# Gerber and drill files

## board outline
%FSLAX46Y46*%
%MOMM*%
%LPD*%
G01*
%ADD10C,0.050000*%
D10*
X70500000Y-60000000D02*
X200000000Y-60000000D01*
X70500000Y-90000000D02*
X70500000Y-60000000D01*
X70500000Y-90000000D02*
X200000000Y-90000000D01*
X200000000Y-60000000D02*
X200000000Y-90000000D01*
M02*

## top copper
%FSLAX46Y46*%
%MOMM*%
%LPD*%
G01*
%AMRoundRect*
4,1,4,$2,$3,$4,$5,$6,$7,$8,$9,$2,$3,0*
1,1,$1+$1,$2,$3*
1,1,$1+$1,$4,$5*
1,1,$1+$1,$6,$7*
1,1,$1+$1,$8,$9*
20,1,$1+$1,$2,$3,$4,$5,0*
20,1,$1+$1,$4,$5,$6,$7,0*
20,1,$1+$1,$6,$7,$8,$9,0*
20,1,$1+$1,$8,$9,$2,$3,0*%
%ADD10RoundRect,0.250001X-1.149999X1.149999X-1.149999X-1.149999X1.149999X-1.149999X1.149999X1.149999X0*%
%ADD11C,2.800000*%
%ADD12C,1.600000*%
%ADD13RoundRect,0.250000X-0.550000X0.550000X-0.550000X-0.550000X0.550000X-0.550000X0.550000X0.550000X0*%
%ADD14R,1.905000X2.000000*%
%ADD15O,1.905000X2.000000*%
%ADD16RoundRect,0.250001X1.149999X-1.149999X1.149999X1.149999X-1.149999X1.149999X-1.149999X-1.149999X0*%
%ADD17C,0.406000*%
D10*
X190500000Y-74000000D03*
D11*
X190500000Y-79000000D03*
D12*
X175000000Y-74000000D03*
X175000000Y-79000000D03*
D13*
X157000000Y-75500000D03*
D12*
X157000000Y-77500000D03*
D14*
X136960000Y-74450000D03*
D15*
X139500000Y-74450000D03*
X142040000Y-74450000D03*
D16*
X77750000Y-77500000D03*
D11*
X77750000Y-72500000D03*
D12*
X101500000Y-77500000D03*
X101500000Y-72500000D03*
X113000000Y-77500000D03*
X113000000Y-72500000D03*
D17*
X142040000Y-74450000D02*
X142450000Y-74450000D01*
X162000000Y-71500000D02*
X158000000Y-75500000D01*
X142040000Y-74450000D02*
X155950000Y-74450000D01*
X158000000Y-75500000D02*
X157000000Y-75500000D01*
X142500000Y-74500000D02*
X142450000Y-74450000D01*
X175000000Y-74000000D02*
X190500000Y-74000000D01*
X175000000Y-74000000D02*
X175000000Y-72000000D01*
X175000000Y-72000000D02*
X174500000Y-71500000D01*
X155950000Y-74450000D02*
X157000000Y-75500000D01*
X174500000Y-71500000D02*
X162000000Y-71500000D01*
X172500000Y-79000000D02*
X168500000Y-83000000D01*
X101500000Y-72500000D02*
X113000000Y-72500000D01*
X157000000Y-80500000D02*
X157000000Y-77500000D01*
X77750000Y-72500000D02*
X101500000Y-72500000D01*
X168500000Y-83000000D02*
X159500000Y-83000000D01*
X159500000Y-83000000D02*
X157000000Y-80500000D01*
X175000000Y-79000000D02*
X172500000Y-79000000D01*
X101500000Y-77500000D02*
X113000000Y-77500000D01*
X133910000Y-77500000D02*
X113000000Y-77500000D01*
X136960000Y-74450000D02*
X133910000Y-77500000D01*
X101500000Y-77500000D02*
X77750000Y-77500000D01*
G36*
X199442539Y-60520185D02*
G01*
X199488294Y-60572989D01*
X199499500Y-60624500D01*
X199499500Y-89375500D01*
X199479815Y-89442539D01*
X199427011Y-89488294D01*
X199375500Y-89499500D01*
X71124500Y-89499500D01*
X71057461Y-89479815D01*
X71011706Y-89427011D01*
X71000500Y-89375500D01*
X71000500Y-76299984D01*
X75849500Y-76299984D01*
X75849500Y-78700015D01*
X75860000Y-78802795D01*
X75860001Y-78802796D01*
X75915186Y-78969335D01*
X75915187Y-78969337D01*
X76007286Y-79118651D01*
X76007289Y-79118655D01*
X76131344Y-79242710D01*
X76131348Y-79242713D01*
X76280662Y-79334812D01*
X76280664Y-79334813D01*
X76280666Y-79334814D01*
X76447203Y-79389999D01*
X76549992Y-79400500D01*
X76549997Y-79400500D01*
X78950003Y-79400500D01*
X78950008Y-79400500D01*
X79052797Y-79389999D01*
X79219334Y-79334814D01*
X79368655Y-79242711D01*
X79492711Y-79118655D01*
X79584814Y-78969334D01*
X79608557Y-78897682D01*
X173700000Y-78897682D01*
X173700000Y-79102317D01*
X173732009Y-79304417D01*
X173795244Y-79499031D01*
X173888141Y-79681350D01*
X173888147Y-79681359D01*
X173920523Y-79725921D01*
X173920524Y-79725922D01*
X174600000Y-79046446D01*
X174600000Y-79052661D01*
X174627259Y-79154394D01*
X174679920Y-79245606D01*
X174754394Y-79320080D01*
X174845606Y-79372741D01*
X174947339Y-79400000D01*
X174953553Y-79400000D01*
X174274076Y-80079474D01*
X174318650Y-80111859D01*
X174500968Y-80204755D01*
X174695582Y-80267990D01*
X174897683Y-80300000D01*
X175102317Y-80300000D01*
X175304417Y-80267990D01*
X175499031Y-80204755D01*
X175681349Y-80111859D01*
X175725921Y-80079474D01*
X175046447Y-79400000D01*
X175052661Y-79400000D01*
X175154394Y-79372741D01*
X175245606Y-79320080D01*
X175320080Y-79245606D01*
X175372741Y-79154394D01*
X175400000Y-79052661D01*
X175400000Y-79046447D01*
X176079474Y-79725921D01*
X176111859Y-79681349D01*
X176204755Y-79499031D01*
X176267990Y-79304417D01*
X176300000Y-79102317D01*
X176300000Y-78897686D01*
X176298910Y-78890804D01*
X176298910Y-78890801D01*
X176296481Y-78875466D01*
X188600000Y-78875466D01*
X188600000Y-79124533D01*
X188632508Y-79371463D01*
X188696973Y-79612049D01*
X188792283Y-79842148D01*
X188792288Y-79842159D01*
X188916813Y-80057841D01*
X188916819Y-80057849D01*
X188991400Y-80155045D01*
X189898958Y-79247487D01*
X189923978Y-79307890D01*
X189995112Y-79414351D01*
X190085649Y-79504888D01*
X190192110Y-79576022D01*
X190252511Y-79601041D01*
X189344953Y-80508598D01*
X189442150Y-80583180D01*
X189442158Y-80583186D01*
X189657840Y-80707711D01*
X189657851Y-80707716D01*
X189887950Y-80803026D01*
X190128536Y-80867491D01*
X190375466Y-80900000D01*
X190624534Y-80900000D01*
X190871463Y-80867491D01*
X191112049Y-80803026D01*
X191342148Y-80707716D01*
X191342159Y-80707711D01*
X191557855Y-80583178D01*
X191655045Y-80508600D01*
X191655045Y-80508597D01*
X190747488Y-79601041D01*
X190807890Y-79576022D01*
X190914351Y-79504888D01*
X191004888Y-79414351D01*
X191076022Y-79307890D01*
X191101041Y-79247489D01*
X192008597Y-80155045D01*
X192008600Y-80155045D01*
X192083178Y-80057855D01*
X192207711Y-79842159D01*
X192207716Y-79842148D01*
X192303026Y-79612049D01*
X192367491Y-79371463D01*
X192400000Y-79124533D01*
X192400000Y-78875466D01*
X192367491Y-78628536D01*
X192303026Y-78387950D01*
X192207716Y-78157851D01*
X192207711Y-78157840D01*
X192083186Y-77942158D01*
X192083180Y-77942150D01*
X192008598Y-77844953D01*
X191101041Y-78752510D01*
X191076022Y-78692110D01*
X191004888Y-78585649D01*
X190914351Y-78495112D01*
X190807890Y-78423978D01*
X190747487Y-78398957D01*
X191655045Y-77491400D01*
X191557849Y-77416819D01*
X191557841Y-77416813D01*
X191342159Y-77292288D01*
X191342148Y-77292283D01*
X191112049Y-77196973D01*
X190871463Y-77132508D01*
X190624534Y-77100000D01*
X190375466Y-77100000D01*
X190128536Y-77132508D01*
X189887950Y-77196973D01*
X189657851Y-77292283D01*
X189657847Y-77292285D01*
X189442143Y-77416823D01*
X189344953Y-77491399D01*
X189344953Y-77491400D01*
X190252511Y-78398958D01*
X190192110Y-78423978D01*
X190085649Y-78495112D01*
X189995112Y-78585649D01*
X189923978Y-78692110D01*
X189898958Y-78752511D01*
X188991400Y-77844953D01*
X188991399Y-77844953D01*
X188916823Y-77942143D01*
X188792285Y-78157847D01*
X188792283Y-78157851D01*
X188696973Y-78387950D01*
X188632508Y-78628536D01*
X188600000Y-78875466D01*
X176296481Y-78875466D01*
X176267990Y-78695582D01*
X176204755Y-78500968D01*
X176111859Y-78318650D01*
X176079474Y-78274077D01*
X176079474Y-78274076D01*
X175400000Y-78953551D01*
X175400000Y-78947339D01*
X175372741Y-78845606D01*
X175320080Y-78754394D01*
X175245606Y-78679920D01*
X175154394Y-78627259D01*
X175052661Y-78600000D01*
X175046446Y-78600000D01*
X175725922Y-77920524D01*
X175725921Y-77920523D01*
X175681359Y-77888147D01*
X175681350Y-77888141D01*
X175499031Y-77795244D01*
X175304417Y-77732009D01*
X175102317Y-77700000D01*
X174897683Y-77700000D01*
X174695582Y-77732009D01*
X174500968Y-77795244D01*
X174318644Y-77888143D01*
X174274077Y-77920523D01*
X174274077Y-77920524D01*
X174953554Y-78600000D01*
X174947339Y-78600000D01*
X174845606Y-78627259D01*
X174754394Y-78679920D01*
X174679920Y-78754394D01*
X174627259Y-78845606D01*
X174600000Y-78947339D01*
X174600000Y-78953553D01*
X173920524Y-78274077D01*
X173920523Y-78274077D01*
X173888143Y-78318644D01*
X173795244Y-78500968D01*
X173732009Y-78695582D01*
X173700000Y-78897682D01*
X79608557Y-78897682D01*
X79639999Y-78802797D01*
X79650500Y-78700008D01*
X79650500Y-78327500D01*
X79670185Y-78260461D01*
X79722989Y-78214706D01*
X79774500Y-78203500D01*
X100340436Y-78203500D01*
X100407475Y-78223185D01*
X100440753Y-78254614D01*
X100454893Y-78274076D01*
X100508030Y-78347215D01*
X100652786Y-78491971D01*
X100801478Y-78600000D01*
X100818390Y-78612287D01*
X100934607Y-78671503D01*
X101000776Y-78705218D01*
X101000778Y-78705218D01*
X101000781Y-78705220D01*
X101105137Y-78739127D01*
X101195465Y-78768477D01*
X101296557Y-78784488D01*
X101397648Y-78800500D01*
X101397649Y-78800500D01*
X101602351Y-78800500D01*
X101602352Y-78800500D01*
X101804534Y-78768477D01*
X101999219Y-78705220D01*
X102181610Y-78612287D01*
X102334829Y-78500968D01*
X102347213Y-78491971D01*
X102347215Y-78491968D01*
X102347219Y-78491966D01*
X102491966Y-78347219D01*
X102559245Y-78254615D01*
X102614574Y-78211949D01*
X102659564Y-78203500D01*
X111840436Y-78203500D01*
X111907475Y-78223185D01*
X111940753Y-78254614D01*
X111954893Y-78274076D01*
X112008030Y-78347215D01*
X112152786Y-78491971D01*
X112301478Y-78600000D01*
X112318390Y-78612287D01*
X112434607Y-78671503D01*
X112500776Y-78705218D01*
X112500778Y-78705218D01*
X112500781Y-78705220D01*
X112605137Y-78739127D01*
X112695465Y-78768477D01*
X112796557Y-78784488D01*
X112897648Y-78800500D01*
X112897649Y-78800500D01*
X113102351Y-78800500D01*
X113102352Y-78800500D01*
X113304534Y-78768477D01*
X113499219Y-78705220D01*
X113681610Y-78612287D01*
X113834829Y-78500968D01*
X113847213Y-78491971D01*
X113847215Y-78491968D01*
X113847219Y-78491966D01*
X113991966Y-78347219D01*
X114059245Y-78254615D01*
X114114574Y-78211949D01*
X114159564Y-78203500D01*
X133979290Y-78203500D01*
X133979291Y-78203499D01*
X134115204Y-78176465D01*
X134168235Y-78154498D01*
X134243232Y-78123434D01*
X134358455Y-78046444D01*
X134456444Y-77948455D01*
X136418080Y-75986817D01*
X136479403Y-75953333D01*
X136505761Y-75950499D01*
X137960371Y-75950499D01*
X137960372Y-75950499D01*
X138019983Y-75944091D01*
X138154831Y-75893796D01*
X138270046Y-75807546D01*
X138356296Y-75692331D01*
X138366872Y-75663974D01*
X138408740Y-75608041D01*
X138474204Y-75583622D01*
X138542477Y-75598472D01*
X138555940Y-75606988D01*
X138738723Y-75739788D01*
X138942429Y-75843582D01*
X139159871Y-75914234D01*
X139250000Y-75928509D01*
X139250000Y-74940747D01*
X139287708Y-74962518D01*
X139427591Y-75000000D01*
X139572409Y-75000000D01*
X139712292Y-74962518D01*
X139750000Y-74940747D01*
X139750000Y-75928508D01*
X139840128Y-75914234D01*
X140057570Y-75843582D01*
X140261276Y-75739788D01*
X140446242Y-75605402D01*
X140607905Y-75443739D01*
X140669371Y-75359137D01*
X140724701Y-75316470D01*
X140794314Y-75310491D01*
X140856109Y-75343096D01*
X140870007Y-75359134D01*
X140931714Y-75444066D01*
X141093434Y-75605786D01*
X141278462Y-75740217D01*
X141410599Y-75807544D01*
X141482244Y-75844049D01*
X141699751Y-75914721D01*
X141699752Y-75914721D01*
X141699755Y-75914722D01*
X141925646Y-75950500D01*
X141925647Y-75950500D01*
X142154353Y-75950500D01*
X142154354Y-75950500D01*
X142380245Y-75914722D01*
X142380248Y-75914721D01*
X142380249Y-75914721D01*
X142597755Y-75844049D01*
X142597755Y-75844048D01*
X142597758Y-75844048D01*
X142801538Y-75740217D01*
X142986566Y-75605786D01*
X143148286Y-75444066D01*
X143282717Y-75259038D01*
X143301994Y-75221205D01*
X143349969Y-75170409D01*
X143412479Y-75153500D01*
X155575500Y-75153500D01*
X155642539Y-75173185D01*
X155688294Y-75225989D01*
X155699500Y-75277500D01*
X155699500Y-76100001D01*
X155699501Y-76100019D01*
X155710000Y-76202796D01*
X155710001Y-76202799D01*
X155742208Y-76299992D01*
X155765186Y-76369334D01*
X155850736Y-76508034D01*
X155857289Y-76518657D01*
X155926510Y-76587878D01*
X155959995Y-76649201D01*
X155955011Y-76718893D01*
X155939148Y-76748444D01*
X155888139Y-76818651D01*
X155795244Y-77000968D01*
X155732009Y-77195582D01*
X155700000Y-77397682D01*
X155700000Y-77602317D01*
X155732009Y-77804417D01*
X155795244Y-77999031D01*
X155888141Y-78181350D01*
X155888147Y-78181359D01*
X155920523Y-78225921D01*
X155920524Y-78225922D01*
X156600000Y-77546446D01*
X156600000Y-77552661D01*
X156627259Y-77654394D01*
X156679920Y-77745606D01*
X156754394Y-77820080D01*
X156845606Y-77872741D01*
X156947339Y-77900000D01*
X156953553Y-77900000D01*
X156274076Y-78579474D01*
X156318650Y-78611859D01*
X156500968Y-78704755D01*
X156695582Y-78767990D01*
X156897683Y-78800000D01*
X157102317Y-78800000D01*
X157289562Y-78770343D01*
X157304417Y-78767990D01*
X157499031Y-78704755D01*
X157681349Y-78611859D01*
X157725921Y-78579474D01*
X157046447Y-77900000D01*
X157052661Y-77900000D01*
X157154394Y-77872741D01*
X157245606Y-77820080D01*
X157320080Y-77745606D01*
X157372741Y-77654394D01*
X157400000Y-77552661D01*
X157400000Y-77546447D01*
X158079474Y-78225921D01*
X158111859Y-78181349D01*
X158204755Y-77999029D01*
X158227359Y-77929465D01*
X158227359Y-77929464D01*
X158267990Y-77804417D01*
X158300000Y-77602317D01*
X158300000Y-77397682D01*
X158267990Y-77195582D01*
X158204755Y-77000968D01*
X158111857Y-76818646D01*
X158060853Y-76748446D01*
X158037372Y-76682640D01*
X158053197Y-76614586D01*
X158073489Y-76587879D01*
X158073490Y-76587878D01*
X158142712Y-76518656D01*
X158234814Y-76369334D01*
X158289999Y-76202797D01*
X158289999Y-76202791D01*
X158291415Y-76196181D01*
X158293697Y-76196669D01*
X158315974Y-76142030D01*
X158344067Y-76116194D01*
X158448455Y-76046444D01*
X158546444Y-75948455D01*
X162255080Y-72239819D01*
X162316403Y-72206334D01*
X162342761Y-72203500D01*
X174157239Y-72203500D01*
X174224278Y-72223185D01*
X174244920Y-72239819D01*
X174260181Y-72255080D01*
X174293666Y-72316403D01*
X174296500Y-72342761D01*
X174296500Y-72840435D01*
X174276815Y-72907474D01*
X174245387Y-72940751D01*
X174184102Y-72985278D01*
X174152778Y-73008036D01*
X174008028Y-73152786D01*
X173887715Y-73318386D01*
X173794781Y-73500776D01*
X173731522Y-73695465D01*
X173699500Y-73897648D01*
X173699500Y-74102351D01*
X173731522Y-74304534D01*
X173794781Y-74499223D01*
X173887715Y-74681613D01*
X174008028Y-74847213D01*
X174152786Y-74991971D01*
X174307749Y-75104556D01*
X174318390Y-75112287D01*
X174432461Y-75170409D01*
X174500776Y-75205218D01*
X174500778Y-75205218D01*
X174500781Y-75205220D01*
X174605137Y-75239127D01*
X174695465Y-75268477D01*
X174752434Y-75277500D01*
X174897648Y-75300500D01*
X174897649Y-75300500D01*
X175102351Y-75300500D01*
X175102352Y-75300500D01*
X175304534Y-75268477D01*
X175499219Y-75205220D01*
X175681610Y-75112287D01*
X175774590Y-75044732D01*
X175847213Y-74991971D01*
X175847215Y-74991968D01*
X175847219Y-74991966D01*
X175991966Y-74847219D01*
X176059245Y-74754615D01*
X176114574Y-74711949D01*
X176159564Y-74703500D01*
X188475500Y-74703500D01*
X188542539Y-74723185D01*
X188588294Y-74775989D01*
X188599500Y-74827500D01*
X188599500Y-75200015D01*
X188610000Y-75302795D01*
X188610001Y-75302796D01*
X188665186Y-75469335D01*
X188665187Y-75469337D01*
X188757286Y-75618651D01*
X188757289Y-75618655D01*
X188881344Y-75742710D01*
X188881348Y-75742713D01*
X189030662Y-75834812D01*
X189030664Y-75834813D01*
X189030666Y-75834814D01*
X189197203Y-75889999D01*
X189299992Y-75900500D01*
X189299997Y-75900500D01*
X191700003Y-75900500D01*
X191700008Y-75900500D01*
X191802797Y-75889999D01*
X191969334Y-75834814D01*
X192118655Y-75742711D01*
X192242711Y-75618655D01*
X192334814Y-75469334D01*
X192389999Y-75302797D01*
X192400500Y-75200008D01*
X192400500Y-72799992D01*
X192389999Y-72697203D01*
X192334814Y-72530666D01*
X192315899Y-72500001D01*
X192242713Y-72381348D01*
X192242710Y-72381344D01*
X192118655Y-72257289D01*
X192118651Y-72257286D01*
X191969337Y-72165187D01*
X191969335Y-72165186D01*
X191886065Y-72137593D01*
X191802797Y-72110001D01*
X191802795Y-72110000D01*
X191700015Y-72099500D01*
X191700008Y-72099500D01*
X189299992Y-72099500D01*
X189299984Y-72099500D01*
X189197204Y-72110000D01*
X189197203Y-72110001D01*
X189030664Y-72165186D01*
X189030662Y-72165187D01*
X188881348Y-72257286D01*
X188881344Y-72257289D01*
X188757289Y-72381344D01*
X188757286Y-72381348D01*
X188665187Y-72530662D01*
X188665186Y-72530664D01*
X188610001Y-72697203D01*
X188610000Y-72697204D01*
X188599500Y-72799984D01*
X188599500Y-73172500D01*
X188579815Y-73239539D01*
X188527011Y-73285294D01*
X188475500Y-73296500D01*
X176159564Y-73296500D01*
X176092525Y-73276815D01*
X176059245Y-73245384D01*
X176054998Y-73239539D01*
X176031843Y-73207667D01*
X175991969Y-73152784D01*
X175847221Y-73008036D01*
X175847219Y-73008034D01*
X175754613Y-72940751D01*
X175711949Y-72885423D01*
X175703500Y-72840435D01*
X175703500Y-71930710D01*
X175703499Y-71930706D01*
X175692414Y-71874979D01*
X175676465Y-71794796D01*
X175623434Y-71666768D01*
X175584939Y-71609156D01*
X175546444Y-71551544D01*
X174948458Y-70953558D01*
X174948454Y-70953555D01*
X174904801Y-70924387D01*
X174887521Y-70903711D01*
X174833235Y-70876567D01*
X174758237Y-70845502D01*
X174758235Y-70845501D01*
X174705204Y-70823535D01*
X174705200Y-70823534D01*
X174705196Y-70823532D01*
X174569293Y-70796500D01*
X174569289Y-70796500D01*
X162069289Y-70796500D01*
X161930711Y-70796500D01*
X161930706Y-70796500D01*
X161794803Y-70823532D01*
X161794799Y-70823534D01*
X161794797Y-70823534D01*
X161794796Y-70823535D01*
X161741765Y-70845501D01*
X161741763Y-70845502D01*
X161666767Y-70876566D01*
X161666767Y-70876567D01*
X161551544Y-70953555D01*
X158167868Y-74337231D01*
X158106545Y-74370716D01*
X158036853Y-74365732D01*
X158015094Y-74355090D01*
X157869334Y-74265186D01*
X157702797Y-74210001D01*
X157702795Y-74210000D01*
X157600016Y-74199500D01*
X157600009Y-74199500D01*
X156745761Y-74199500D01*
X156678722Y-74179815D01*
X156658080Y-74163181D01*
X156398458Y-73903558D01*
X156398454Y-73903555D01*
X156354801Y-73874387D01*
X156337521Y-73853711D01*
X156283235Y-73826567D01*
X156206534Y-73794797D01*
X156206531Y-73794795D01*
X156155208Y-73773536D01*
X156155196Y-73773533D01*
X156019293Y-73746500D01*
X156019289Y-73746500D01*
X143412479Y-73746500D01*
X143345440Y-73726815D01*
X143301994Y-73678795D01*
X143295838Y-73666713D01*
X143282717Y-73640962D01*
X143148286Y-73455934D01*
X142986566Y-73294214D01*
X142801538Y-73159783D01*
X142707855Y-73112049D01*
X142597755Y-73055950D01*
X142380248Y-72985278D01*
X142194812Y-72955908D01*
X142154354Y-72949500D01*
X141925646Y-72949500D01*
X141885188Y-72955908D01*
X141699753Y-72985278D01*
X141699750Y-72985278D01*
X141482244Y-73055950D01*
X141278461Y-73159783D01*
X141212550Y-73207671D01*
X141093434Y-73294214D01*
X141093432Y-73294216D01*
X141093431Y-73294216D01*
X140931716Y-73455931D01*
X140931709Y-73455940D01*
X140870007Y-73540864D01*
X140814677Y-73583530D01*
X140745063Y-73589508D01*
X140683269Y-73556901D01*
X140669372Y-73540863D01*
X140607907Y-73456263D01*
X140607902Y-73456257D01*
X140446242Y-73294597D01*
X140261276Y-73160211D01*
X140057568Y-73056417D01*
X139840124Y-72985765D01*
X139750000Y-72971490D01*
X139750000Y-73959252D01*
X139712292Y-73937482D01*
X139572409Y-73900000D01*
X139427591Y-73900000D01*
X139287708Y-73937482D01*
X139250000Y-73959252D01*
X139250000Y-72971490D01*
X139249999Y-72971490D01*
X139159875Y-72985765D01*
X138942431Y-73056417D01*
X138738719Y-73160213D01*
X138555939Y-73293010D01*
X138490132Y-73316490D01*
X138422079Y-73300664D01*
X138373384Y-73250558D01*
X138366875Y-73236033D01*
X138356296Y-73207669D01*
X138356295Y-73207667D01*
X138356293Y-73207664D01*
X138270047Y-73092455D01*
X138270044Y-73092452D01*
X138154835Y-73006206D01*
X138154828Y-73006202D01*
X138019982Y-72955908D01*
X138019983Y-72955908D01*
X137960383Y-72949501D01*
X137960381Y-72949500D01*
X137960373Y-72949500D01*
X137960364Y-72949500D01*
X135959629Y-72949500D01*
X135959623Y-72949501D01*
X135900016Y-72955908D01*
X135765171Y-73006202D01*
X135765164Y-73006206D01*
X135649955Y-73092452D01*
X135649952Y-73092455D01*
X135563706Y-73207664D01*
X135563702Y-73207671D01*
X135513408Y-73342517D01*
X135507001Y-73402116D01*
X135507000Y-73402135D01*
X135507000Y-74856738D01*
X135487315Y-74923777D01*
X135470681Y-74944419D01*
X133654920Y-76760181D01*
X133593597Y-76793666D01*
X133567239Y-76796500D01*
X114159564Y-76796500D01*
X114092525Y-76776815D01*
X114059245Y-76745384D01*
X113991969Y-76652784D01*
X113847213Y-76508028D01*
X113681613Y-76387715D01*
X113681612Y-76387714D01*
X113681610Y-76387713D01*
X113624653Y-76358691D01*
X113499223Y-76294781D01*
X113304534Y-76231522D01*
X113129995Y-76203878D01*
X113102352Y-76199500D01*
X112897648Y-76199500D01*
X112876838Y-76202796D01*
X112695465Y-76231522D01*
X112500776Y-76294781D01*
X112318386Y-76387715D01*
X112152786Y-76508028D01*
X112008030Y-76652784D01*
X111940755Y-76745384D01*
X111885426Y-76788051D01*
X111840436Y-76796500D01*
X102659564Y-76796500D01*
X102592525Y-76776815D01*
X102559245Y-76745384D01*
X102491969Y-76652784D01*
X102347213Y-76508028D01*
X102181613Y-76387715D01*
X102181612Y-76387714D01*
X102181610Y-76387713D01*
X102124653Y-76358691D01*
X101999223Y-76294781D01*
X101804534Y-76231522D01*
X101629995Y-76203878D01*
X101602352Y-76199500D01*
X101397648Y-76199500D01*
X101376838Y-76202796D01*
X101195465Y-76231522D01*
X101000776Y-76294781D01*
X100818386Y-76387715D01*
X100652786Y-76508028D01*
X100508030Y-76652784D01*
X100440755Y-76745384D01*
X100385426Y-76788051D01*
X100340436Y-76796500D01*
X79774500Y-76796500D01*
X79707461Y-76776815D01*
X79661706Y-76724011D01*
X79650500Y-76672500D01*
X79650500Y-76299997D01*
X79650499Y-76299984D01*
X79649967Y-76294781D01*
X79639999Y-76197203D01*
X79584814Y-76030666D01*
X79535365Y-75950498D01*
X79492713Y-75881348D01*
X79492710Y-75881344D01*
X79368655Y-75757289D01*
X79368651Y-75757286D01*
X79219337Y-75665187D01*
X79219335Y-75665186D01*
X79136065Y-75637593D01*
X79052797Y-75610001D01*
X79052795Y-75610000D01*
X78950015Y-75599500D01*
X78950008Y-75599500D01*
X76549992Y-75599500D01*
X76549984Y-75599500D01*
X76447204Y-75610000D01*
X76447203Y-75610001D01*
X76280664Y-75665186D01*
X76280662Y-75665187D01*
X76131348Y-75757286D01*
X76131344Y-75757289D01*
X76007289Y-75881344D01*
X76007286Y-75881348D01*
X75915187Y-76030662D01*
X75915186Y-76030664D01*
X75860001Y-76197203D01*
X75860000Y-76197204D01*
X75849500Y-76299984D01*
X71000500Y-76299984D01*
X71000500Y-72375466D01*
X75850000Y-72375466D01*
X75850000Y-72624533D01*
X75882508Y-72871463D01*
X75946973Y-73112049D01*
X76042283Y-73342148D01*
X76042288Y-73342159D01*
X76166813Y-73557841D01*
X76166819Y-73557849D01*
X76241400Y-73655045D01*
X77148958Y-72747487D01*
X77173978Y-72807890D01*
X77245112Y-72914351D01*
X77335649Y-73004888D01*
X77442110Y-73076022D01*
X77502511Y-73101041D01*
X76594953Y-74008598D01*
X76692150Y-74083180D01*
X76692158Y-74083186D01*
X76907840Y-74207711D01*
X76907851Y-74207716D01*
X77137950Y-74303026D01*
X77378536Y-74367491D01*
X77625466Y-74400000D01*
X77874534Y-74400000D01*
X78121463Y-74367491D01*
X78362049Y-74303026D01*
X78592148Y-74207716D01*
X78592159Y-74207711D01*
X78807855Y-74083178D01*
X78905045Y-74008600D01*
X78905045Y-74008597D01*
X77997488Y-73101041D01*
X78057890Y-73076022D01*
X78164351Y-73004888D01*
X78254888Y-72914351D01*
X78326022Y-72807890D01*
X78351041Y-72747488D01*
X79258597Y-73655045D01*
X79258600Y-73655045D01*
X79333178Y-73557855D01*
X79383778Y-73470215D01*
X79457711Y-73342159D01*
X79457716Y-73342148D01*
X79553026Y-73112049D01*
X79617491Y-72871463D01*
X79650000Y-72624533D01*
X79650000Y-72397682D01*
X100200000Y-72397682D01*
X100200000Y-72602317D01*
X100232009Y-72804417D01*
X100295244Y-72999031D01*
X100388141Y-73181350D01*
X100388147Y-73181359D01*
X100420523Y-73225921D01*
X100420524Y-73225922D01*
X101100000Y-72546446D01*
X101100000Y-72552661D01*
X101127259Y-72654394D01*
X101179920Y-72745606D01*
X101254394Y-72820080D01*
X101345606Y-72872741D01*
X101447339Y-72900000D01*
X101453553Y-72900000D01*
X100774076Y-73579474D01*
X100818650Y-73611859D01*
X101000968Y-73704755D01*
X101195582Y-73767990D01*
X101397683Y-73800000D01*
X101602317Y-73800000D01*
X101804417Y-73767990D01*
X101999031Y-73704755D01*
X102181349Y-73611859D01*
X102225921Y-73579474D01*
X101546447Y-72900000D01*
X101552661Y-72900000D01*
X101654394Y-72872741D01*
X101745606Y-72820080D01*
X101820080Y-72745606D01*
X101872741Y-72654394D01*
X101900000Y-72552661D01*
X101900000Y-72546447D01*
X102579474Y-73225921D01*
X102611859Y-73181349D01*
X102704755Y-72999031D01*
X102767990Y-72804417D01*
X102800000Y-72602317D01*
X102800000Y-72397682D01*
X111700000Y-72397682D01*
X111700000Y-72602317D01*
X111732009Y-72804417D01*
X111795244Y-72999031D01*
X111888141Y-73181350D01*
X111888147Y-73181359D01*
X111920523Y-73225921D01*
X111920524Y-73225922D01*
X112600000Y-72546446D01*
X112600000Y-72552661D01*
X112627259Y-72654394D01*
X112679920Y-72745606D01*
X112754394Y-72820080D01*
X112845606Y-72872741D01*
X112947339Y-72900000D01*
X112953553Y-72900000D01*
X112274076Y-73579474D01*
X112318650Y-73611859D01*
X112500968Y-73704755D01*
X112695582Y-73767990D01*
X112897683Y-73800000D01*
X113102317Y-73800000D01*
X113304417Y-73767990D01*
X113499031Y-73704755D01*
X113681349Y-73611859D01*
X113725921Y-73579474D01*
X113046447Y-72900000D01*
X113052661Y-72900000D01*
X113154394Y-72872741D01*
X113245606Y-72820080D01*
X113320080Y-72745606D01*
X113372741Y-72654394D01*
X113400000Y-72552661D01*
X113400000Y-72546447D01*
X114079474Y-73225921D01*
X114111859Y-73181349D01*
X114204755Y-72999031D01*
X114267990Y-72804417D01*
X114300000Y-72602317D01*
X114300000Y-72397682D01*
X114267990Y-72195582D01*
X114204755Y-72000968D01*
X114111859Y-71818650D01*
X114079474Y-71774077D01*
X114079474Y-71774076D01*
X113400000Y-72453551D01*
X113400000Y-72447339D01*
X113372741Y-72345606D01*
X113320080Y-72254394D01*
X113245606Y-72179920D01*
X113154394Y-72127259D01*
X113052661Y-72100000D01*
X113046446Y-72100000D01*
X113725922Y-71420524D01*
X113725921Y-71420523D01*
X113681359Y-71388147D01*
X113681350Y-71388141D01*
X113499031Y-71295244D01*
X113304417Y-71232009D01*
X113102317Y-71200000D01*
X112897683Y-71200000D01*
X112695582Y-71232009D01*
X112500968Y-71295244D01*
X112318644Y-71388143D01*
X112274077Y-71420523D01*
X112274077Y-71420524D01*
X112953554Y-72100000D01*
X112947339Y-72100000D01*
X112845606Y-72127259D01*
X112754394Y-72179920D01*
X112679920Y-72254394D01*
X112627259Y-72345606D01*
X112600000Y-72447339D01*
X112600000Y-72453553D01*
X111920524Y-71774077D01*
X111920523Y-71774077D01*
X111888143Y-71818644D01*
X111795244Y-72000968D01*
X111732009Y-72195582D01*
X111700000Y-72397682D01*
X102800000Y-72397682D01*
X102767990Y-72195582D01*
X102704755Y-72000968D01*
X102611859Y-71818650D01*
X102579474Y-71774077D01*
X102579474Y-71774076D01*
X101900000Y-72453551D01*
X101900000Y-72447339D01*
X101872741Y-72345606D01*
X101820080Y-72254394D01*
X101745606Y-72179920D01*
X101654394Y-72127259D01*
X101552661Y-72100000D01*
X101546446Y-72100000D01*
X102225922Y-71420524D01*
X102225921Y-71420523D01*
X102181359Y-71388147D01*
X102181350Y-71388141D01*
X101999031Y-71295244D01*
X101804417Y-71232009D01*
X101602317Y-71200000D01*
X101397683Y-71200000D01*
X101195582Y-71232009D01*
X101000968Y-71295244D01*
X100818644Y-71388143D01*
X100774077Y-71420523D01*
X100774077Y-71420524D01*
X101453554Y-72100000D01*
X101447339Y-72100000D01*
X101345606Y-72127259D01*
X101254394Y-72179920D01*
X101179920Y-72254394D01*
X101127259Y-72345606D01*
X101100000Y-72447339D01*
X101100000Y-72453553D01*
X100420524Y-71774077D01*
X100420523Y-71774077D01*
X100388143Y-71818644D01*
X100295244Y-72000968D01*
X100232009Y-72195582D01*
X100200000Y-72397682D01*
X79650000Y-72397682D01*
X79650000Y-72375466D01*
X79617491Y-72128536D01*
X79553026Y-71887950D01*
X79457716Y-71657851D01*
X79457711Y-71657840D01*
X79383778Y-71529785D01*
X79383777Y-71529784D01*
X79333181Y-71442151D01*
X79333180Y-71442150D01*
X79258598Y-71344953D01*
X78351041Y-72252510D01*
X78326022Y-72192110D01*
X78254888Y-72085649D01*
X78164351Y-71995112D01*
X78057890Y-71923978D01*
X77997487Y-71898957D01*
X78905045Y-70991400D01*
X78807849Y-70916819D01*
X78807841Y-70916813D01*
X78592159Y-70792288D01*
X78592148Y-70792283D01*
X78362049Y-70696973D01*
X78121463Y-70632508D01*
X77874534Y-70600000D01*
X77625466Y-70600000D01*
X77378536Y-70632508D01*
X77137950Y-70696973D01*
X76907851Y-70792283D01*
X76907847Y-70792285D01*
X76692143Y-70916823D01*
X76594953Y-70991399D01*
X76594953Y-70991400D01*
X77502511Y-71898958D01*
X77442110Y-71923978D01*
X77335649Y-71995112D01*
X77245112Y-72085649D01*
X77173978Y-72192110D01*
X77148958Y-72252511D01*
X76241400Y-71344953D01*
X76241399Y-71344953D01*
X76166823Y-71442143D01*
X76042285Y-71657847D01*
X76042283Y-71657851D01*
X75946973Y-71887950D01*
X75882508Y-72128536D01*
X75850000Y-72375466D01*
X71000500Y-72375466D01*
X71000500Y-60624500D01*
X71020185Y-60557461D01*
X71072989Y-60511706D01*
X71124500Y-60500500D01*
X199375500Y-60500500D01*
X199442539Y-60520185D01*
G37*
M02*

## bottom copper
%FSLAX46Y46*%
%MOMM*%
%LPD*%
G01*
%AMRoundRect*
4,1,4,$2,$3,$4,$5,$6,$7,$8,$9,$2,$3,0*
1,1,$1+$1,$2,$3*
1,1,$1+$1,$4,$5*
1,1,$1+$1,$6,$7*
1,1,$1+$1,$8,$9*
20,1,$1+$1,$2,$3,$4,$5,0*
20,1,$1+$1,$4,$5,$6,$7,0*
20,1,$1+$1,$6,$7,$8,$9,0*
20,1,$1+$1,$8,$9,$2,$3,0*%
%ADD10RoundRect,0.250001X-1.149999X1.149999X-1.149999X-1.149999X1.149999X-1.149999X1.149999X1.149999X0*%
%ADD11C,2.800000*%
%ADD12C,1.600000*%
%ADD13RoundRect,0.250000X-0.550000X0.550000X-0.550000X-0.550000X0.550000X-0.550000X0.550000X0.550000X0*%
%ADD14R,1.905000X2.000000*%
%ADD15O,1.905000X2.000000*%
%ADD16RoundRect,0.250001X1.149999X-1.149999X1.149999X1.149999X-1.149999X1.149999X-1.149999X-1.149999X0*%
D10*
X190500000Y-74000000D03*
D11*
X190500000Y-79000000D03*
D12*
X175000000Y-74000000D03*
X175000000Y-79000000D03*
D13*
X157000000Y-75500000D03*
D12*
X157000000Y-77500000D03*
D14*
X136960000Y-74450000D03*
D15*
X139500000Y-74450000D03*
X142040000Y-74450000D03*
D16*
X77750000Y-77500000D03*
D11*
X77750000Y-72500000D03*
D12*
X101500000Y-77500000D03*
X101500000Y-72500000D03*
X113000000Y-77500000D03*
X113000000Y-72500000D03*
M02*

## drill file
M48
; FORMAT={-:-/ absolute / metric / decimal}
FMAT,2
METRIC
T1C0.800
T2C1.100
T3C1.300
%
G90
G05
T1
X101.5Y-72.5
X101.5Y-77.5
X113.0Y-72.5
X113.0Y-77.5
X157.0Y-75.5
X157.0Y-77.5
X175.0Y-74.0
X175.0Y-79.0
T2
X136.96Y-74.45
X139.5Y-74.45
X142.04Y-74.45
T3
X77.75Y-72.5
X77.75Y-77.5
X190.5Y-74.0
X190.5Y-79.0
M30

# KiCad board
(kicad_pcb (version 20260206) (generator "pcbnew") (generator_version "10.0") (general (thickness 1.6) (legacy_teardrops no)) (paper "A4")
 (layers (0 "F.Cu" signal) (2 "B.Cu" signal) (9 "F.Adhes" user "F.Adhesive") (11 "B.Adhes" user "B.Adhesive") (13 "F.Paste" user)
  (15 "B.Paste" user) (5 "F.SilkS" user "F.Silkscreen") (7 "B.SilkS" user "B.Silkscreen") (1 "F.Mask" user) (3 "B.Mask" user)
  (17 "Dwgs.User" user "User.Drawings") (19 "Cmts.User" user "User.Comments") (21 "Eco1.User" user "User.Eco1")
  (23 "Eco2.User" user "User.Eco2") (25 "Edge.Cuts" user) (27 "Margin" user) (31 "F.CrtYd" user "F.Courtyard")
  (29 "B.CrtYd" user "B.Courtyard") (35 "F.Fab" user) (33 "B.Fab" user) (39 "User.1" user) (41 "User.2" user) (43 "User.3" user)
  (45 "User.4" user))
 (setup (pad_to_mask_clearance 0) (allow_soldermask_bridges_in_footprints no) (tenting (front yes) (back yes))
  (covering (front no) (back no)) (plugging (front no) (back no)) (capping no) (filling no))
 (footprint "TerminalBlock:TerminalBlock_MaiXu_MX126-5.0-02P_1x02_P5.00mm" (layer "F.Cu") (at 190.5 74 -90)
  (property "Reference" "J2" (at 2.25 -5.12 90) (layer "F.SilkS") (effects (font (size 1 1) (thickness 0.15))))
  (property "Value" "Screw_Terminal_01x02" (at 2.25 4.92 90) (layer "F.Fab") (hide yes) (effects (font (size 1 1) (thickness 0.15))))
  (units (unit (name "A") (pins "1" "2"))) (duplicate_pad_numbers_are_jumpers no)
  (pad "1" thru_hole roundrect (at 0 0 270) (size 2.8 2.8) (drill 1.3) (layers "*.Cu" "*.Mask") (remove_unused_layers no)
   (roundrect_rratio 0.089286) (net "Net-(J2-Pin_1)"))
  (pad "2" thru_hole circle (at 5 0 270) (size 2.8 2.8) (drill 1.3) (layers "*.Cu" "*.Mask") (remove_unused_layers no) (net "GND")))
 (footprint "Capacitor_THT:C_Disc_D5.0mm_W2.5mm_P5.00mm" (layer "F.Cu") (at 175 74 -90)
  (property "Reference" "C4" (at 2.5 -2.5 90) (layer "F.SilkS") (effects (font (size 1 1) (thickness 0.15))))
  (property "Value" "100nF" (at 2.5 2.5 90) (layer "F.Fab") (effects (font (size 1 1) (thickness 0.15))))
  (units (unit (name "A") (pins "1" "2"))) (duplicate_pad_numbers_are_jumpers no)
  (pad "1" thru_hole circle (at 0 0 270) (size 1.6 1.6) (drill 0.8) (layers "*.Cu" "*.Mask") (remove_unused_layers no)
   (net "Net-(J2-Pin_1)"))
  (pad "2" thru_hole circle (at 5 0 270) (size 1.6 1.6) (drill 0.8) (layers "*.Cu" "*.Mask") (remove_unused_layers no) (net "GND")))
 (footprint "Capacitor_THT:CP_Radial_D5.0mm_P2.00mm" (layer "F.Cu") (at 157 75.5 -90)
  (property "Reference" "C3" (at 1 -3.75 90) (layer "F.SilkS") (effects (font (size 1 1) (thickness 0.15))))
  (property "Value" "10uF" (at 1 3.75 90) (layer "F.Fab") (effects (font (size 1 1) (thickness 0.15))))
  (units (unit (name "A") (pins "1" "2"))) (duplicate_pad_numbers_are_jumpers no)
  (pad "1" thru_hole roundrect (at 0 0 270) (size 1.6 1.6) (drill 0.8) (layers "*.Cu" "*.Mask") (remove_unused_layers no)
   (roundrect_rratio 0.15625) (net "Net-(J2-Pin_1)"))
  (pad "2" thru_hole circle (at 2 0 270) (size 1.6 1.6) (drill 0.8) (layers "*.Cu" "*.Mask") (remove_unused_layers no) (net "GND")))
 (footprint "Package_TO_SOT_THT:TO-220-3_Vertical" (layer "F.Cu") (at 136.96 74.45)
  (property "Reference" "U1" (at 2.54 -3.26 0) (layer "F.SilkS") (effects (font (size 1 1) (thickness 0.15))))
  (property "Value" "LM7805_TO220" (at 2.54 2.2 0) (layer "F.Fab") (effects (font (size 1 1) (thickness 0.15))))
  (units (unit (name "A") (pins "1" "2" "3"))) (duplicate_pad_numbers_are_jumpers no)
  (pad "1" thru_hole rect (at 0 0) (size 1.905 2) (drill 1.1) (layers "*.Cu" "*.Mask") (remove_unused_layers no) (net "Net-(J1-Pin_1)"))
  (pad "2" thru_hole oval (at 2.54 0) (size 1.905 2) (drill 1.1) (layers "*.Cu" "*.Mask") (remove_unused_layers no) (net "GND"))
  (pad "3" thru_hole oval (at 5.08 0) (size 1.905 2) (drill 1.1) (layers "*.Cu" "*.Mask") (remove_unused_layers no) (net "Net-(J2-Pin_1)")))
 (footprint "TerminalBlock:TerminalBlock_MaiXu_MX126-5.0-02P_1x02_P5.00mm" (layer "F.Cu") (at 77.75 77.5 90)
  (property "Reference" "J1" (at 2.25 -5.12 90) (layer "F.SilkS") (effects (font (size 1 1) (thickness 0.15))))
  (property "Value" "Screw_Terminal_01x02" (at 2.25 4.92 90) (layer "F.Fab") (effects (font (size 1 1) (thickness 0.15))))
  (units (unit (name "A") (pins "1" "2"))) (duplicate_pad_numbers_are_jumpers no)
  (pad "1" thru_hole roundrect (at 0 0 90) (size 2.8 2.8) (drill 1.3) (layers "*.Cu" "*.Mask") (remove_unused_layers no)
   (roundrect_rratio 0.089286) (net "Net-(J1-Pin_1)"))
  (pad "2" thru_hole circle (at 5 0 90) (size 2.8 2.8) (drill 1.3) (layers "*.Cu" "*.Mask") (remove_unused_layers no) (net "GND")))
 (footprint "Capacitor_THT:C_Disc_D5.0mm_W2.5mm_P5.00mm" (layer "F.Cu") (at 101.5 77.5 90)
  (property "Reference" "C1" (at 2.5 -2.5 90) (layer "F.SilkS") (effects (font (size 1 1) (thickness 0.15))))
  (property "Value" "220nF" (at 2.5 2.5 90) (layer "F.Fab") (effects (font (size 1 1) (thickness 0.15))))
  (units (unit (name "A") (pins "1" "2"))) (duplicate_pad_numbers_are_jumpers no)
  (pad "1" thru_hole circle (at 0 0 90) (size 1.6 1.6) (drill 0.8) (layers "*.Cu" "*.Mask") (remove_unused_layers no) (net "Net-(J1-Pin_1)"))
  (pad "2" thru_hole circle (at 5 0 90) (size 1.6 1.6) (drill 0.8) (layers "*.Cu" "*.Mask") (remove_unused_layers no) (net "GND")))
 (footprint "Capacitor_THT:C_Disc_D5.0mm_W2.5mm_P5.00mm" (layer "F.Cu") (at 113 77.5 90)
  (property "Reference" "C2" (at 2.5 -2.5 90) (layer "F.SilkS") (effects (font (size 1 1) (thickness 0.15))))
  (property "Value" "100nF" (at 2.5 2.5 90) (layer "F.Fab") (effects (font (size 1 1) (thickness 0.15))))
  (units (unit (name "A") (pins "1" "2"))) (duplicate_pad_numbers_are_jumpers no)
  (pad "1" thru_hole circle (at 0 0 90) (size 1.6 1.6) (drill 0.8) (layers "*.Cu" "*.Mask") (remove_unused_layers no) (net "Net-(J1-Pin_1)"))
  (pad "2" thru_hole circle (at 5 0 90) (size 1.6 1.6) (drill 0.8) (layers "*.Cu" "*.Mask") (remove_unused_layers no) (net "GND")))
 (gr_line (start 70.5 60) (end 200 60) (stroke (width 0.05) (type default)) (layer "Edge.Cuts"))
 (gr_line (start 70.5 90) (end 70.5 60) (stroke (width 0.05) (type default)) (layer "Edge.Cuts"))
 (gr_line (start 70.5 90) (end 200 90) (stroke (width 0.05) (type default)) (layer "Edge.Cuts"))
 (gr_line (start 200 60) (end 200 90) (stroke (width 0.05) (type default)) (layer "Edge.Cuts"))
 (segment (start 142.04 74.45) (end 142.45 74.45) (width 0.406) (layer "F.Cu") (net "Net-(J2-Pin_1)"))
 (segment (start 162 71.5) (end 158 75.5) (width 0.406) (layer "F.Cu") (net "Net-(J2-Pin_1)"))
 (segment (start 142.04 74.45) (end 155.95 74.45) (width 0.406) (layer "F.Cu") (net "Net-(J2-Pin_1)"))
 (segment (start 158 75.5) (end 157 75.5) (width 0.406) (layer "F.Cu") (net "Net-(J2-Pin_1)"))
 (segment (start 142.5 74.5) (end 142.45 74.45) (width 0.406) (layer "F.Cu") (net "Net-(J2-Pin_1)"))
 (segment (start 175 74) (end 190.5 74) (width 0.406) (layer "F.Cu") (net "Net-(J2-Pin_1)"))
 (segment (start 175 74) (end 175 72) (width 0.406) (layer "F.Cu") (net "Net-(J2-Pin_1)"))
 (segment (start 175 72) (end 174.5 71.5) (width 0.406) (layer "F.Cu") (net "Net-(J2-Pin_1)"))
 (segment (start 155.95 74.45) (end 157 75.5) (width 0.406) (layer "F.Cu") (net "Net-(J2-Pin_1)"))
 (segment (start 174.5 71.5) (end 162 71.5) (width 0.406) (layer "F.Cu") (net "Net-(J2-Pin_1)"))
 (segment (start 172.5 79) (end 168.5 83) (width 0.406) (layer "F.Cu") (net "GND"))
 (segment (start 101.5 72.5) (end 113 72.5) (width 0.406) (layer "F.Cu") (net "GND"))
 (segment (start 157 80.5) (end 157 77.5) (width 0.406) (layer "F.Cu") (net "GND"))
 (segment (start 77.75 72.5) (end 101.5 72.5) (width 0.406) (layer "F.Cu") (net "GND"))
 (segment (start 168.5 83) (end 159.5 83) (width 0.406) (layer "F.Cu") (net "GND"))
 (segment (start 159.5 83) (end 157 80.5) (width 0.406) (layer "F.Cu") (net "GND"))
 (segment (start 175 79) (end 172.5 79) (width 0.406) (layer "F.Cu") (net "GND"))
 (segment (start 101.5 77.5) (end 113 77.5) (width 0.406) (layer "F.Cu") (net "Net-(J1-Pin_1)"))
 (segment (start 133.91 77.5) (end 113 77.5) (width 0.406) (layer "F.Cu") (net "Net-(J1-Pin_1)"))
 (segment (start 136.96 74.45) (end 133.91 77.5) (width 0.406) (layer "F.Cu") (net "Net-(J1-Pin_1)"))
 (segment (start 101.5 77.5) (end 77.75 77.5) (width 0.406) (layer "F.Cu") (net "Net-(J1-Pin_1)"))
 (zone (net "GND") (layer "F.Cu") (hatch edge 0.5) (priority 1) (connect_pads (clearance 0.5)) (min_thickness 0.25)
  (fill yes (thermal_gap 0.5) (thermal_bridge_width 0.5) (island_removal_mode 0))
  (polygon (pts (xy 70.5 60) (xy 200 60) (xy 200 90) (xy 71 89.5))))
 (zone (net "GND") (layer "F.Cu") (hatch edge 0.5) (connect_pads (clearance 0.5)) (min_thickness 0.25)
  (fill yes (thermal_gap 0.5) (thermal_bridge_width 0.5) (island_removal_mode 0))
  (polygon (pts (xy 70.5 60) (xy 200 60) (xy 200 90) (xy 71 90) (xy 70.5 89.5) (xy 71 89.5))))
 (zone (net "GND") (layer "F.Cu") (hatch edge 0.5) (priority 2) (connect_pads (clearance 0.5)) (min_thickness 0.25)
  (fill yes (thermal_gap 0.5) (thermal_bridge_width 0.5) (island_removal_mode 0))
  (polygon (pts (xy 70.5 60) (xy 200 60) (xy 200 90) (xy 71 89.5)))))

